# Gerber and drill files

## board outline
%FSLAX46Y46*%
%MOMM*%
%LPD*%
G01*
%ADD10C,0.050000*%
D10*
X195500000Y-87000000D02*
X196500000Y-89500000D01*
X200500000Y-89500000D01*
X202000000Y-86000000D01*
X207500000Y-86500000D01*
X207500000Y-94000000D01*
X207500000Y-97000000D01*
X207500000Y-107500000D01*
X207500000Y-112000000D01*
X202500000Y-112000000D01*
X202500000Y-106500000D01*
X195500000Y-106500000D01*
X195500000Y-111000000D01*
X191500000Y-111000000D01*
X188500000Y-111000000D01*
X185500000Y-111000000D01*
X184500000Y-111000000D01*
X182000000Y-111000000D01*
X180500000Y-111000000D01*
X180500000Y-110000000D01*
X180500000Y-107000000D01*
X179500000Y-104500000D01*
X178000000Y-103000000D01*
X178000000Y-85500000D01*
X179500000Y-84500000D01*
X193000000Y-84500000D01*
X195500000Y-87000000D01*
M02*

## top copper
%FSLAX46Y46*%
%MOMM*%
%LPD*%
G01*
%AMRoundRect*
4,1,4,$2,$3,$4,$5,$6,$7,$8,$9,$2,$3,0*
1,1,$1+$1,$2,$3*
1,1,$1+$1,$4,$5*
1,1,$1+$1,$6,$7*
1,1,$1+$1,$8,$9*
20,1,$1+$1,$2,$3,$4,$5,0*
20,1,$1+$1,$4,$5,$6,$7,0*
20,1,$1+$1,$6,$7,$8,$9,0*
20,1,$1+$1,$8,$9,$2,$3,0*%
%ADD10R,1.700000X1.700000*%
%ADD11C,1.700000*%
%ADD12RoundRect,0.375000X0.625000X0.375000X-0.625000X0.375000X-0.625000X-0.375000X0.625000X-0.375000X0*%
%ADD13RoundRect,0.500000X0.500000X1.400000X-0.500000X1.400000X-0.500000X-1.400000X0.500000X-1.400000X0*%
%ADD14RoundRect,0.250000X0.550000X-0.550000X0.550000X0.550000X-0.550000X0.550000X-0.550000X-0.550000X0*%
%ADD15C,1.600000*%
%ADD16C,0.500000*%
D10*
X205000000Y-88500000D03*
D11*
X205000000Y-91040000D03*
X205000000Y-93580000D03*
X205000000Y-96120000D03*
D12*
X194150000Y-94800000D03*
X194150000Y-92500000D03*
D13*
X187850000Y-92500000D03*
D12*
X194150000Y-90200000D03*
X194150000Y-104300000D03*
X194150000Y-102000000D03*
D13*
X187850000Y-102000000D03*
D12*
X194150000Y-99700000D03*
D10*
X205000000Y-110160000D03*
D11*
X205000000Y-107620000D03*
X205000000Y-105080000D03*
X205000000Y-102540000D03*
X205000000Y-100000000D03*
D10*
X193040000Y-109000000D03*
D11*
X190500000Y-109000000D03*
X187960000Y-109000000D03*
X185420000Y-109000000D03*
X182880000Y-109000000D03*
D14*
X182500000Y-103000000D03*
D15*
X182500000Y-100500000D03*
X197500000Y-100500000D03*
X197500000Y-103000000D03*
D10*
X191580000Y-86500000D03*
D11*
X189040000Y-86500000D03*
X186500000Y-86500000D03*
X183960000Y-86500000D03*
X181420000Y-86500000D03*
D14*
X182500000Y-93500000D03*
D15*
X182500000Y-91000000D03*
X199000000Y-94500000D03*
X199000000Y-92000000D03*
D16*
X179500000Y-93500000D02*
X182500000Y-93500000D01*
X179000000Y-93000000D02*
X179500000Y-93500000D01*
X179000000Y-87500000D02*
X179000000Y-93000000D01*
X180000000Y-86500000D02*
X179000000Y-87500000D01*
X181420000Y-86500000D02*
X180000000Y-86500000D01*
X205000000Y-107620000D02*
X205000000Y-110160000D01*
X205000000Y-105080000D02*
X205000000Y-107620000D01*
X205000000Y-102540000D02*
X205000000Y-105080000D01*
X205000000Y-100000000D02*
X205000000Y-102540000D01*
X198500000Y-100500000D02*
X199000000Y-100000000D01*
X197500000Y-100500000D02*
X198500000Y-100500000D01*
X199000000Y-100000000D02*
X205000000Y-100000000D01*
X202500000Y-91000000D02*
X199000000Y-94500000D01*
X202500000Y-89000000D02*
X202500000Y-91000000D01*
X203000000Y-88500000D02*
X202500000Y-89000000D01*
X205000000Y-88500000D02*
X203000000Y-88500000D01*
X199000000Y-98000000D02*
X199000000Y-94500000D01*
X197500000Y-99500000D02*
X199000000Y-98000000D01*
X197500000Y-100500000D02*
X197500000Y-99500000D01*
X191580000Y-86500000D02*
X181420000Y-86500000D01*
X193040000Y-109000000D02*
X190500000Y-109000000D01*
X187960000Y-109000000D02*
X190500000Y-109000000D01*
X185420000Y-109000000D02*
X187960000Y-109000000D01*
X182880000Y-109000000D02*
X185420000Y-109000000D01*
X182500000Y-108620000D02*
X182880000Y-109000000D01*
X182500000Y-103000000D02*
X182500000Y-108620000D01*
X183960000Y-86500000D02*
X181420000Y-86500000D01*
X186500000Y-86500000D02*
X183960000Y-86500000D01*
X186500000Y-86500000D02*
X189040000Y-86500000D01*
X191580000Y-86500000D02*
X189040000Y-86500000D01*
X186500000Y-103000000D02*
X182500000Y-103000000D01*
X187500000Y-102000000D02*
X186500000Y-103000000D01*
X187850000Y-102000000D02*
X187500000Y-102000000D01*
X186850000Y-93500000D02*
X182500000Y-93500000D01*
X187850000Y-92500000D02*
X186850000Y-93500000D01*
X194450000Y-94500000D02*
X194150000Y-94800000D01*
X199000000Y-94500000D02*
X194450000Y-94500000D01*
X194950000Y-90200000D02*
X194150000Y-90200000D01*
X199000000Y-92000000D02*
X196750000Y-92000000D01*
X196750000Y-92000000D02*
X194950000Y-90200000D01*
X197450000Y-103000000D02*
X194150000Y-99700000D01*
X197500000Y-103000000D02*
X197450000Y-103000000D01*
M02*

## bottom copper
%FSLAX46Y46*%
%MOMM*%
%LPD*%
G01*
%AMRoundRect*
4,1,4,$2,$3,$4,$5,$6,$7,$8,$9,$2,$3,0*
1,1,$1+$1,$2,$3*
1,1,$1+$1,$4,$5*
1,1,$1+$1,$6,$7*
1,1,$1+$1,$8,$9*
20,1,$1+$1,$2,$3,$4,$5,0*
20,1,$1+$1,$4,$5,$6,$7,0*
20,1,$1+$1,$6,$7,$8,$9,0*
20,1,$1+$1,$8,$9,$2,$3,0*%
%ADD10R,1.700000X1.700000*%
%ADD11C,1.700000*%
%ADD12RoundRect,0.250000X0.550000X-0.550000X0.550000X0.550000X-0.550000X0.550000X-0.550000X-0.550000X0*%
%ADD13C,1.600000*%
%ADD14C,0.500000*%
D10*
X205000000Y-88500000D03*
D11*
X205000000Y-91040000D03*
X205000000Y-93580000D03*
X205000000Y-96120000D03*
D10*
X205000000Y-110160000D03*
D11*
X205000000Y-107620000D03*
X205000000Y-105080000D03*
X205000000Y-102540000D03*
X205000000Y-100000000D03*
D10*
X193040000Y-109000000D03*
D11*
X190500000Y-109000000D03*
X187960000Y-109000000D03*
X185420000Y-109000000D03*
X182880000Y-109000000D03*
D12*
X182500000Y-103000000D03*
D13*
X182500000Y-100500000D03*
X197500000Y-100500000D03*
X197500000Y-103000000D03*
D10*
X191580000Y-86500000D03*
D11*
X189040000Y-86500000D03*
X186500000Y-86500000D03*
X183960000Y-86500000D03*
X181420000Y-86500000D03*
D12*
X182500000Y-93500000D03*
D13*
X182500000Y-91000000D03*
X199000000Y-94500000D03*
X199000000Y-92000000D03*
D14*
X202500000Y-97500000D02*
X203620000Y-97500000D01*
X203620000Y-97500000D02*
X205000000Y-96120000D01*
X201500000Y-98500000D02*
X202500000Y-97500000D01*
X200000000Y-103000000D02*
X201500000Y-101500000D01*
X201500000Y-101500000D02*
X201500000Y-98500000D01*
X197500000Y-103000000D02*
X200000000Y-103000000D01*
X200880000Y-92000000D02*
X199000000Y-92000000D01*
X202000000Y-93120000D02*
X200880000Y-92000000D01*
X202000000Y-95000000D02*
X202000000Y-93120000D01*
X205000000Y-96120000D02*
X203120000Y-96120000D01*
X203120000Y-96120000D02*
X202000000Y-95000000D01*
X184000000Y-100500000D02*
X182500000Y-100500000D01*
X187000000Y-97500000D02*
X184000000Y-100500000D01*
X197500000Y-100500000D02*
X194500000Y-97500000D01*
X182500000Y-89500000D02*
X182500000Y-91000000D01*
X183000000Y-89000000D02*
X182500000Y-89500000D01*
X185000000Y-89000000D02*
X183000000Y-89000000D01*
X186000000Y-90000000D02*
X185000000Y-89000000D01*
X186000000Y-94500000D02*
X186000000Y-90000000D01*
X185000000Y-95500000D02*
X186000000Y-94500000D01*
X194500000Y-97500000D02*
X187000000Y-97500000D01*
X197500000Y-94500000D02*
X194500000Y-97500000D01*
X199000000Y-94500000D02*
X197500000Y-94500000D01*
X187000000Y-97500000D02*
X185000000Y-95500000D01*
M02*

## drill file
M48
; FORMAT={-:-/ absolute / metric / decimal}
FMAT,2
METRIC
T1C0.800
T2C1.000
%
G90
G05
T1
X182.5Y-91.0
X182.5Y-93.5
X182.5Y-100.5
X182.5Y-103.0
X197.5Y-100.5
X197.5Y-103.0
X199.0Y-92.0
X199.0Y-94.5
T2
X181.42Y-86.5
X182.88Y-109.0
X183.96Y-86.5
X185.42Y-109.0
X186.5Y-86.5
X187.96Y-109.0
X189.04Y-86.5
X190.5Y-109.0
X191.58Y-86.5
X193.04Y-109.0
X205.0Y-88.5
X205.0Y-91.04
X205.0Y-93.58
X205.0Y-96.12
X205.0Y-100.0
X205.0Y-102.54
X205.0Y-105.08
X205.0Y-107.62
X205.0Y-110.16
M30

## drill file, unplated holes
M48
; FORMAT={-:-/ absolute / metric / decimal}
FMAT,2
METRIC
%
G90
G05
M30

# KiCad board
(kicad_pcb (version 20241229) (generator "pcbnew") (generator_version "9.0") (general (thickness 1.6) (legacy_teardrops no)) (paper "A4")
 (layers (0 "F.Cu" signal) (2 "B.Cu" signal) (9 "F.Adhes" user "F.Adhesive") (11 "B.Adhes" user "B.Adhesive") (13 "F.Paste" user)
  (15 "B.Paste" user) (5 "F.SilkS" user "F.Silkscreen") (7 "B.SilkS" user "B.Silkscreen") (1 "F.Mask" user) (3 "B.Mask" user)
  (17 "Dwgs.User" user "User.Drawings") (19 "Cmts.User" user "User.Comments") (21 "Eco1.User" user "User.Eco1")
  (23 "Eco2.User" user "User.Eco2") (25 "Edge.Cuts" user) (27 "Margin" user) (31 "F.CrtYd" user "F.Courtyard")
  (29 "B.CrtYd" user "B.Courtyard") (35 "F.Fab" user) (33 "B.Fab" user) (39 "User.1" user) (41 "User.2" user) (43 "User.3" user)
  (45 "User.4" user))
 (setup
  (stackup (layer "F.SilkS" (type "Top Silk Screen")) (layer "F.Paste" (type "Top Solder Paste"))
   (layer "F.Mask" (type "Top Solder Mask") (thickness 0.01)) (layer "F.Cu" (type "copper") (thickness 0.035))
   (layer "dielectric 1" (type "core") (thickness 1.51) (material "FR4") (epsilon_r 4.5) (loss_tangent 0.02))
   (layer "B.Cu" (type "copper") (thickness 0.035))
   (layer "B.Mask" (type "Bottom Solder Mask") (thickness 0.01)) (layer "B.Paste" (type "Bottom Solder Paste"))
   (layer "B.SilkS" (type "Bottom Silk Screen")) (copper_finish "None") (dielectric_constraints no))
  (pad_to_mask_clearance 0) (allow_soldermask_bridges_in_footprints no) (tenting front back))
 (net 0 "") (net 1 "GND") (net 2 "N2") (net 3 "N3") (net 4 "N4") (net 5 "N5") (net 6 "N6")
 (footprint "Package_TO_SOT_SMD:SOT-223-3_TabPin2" (layer "F.Cu") (at 191 92.5 180)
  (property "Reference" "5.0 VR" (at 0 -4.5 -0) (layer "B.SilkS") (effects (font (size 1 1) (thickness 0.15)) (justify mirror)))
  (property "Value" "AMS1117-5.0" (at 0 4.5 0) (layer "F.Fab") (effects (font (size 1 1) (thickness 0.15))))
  (pad "1" smd roundrect (at -3.15 -2.3 180) (size 2 1.5) (layers "F.Cu" "F.Mask" "F.Paste") (roundrect_rratio 0.25) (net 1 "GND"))
  (pad "2" smd roundrect (at -3.15 0 180) (size 2 1.5) (layers "F.Cu" "F.Mask" "F.Paste") (roundrect_rratio 0.25) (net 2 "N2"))
  (pad "2" smd roundrect (at 3.15 0 180) (size 2 3.8) (layers "F.Cu" "F.Mask" "F.Paste") (roundrect_rratio 0.25) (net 2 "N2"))
  (pad "3" smd roundrect (at -3.15 2.3 180) (size 2 1.5) (layers "F.Cu" "F.Mask" "F.Paste") (roundrect_rratio 0.25) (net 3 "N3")))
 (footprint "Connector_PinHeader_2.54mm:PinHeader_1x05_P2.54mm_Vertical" (layer "F.Cu") (at 205 110.16 180)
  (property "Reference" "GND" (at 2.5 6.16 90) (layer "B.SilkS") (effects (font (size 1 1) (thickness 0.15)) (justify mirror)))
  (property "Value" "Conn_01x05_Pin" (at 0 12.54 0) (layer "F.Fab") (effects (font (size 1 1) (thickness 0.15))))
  (pad "1" thru_hole rect (at 0 0 180) (size 1.7 1.7) (drill 1) (layers "*.Cu" "*.Mask") (remove_unused_layers no) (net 1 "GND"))
  (pad "2" thru_hole circle (at 0 2.54 180) (size 1.7 1.7) (drill 1) (layers "*.Cu" "*.Mask") (remove_unused_layers no) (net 1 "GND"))
  (pad "3" thru_hole circle (at 0 5.08 180) (size 1.7 1.7) (drill 1) (layers "*.Cu" "*.Mask") (remove_unused_layers no) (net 1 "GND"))
  (pad "4" thru_hole circle (at 0 7.62 180) (size 1.7 1.7) (drill 1) (layers "*.Cu" "*.Mask") (remove_unused_layers no) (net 1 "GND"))
  (pad "5" thru_hole circle (at 0 10.16 180) (size 1.7 1.7) (drill 1) (layers "*.Cu" "*.Mask") (remove_unused_layers no) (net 1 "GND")))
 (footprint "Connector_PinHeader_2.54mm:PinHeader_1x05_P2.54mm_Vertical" (layer "F.Cu") (at 193.04 109 -90)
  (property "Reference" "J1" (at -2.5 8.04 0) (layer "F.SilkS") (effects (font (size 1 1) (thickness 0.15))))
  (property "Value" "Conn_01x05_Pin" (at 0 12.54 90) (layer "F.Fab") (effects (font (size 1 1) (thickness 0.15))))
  (pad "1" thru_hole rect (at 0 0 270) (size 1.7 1.7) (drill 1) (layers "*.Cu" "*.Mask") (remove_unused_layers no) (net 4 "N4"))
  (pad "2" thru_hole circle (at 0 2.54 270) (size 1.7 1.7) (drill 1) (layers "*.Cu" "*.Mask") (remove_unused_layers no) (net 4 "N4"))
  (pad "3" thru_hole circle (at 0 5.08 270) (size 1.7 1.7) (drill 1) (layers "*.Cu" "*.Mask") (remove_unused_layers no) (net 4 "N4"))
  (pad "4" thru_hole circle (at 0 7.62 270) (size 1.7 1.7) (drill 1) (layers "*.Cu" "*.Mask") (remove_unused_layers no) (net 4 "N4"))
  (pad "5" thru_hole circle (at 0 10.16 270) (size 1.7 1.7) (drill 1) (layers "*.Cu" "*.Mask") (remove_unused_layers no) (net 4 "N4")))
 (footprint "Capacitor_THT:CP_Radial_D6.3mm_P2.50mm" (layer "F.Cu") (at 182.5 103 90)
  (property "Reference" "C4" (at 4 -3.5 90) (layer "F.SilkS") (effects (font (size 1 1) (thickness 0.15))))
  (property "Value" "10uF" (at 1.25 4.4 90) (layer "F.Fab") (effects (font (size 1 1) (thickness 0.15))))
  (pad "1" thru_hole roundrect (at 0 0 90) (size 1.6 1.6) (drill 0.8) (layers "*.Cu" "*.Mask") (remove_unused_layers no)
   (roundrect_rratio 0.15625) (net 4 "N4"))
  (pad "2" thru_hole circle (at 2.5 0 90) (size 1.6 1.6) (drill 0.8) (layers "*.Cu" "*.Mask") (remove_unused_layers no) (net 1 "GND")))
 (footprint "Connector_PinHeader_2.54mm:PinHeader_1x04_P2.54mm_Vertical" (layer "F.Cu") (at 205 88.5)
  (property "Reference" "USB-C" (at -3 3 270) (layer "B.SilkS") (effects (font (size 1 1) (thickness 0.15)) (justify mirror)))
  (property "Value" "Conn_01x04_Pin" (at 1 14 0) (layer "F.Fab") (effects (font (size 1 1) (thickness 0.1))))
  (pad "1" thru_hole rect (at 0 0) (size 1.7 1.7) (drill 1) (layers "*.Cu" "*.Mask") (remove_unused_layers no) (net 1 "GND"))
  (pad "2" thru_hole circle (at 0 2.54) (size 1.7 1.7) (drill 1) (layers "*.Cu" "*.Mask") (remove_unused_layers no) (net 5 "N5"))
  (pad "3" thru_hole circle (at 0 5.08) (size 1.7 1.7) (drill 1) (layers "*.Cu" "*.Mask") (remove_unused_layers no) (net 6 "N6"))
  (pad "4" thru_hole circle (at 0 7.62) (size 1.7 1.7) (drill 1) (layers "*.Cu" "*.Mask") (remove_unused_layers no) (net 3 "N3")))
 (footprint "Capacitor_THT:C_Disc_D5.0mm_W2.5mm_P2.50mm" (layer "F.Cu") (at 197.5 100.5 -90)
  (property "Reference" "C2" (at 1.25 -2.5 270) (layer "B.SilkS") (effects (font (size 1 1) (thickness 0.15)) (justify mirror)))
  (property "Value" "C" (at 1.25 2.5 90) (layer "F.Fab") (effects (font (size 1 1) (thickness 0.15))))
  (pad "1" thru_hole circle (at 0 0 270) (size 1.6 1.6) (drill 0.8) (layers "*.Cu" "*.Mask") (remove_unused_layers no) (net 1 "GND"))
  (pad "2" thru_hole circle (at 2.5 0 270) (size 1.6 1.6) (drill 0.8) (layers "*.Cu" "*.Mask") (remove_unused_layers no) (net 3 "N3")))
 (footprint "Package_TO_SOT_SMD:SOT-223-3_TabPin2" (layer "F.Cu") (at 191 102 180)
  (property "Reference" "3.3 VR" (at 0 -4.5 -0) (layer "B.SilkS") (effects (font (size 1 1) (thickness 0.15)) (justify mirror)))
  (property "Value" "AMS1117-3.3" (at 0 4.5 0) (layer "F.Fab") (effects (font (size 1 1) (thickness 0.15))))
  (pad "1" smd roundrect (at -3.15 -2.3 180) (size 2 1.5) (layers "F.Cu" "F.Mask" "F.Paste") (roundrect_rratio 0.25) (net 1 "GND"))
  (pad "2" smd roundrect (at -3.15 0 180) (size 2 1.5) (layers "F.Cu" "F.Mask" "F.Paste") (roundrect_rratio 0.25) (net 4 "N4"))
  (pad "2" smd roundrect (at 3.15 0 180) (size 2 3.8) (layers "F.Cu" "F.Mask" "F.Paste") (roundrect_rratio 0.25) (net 4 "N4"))
  (pad "3" smd roundrect (at -3.15 2.3 180) (size 2 1.5) (layers "F.Cu" "F.Mask" "F.Paste") (roundrect_rratio 0.25) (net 3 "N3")))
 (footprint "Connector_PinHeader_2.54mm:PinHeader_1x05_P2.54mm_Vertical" (layer "F.Cu") (at 191.58 86.5 -90)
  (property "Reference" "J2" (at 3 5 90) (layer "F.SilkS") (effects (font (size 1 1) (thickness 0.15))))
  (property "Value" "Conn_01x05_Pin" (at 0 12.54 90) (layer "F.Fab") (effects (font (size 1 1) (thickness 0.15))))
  (pad "1" thru_hole rect (at 0 0 270) (size 1.7 1.7) (drill 1) (layers "*.Cu" "*.Mask") (remove_unused_layers no) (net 2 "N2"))
  (pad "2" thru_hole circle (at 0 2.54 270) (size 1.7 1.7) (drill 1) (layers "*.Cu" "*.Mask") (remove_unused_layers no) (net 2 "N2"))
  (pad "3" thru_hole circle (at 0 5.08 270) (size 1.7 1.7) (drill 1) (layers "*.Cu" "*.Mask") (remove_unused_layers no) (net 2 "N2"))
  (pad "4" thru_hole circle (at 0 7.62 270) (size 1.7 1.7) (drill 1) (layers "*.Cu" "*.Mask") (remove_unused_layers no) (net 2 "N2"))
  (pad "5" thru_hole circle (at 0 10.16 270) (size 1.7 1.7) (drill 1) (layers "*.Cu" "*.Mask") (remove_unused_layers no) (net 2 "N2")))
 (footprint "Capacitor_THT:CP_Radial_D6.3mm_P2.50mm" (layer "F.Cu") (at 182.5 93.5 90)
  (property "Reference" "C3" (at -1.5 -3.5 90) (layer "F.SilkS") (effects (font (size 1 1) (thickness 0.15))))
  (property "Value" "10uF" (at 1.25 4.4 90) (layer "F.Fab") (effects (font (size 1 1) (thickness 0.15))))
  (pad "1" thru_hole roundrect (at 0 0 90) (size 1.6 1.6) (drill 0.8) (layers "*.Cu" "*.Mask") (remove_unused_layers no)
   (roundrect_rratio 0.15625) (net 2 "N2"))
  (pad "2" thru_hole circle (at 2.5 0 90) (size 1.6 1.6) (drill 0.8) (layers "*.Cu" "*.Mask") (remove_unused_layers no) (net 1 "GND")))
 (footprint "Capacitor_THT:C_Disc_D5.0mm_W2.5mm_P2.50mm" (layer "F.Cu") (at 199 94.5 90)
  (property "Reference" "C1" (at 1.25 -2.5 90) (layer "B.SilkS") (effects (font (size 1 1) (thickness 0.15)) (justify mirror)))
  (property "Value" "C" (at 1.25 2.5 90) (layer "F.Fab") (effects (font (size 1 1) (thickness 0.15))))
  (pad "1" thru_hole circle (at 0 0 90) (size 1.6 1.6) (drill 0.8) (layers "*.Cu" "*.Mask") (remove_unused_layers no) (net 1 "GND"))
  (pad "2" thru_hole circle (at 2.5 0 90) (size 1.6 1.6) (drill 0.8) (layers "*.Cu" "*.Mask") (remove_unused_layers no) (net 3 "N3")))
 (gr_poly
  (pts (xy 207.5 86.5) (xy 207.5 94) (xy 207.5 97) (xy 207.5 107.5) (xy 207.5 107.5) (xy 207.5 112) (xy 202.5 112) (xy 202.5 106.5)
   (xy 195.5 106.5) (xy 195.5 111) (xy 191.5 111) (xy 188.5 111) (xy 185.5 111) (xy 184.5 111) (xy 182 111) (xy 180.5 111) (xy 180.5 110)
   (xy 180.5 107) (xy 179.5 104.5) (xy 178 103) (xy 178 85.5) (xy 179.5 84.5) (xy 193 84.5) (xy 195.5 87) (xy 196.5 89.5) (xy 200.5 89.5)
   (xy 202 86))
  (stroke (width 0.05) (type solid)) (fill no) (layer "Edge.Cuts"))
 (segment (start 199 92) (end 196.75 92) (width 0.5) (layer "F.Cu") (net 3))
 (segment (start 194.95 90.2) (end 194.15 90.2) (width 0.5) (layer "F.Cu") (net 3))
 (segment (start 197.45 103) (end 194.15 99.7) (width 0.5) (layer "F.Cu") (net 3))
 (segment (start 197.5 103) (end 197.45 103) (width 0.5) (layer "F.Cu") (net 3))
 (segment (start 196.75 92) (end 194.95 90.2) (width 0.5) (layer "F.Cu") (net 3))
 (segment (start 200.88 92) (end 199 92) (width 0.5) (layer "B.Cu") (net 3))
 (segment (start 202.5 97.5) (end 203.62 97.5) (width 0.5) (layer "B.Cu") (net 3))
 (segment (start 197.5 103) (end 200 103) (width 0.5) (layer "B.Cu") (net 3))
 (segment (start 200 103) (end 201.5 101.5) (width 0.5) (layer "B.Cu") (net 3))
 (segment (start 202 93.12) (end 200.88 92) (width 0.5) (layer "B.Cu") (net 3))
 (segment (start 202 95) (end 202 93.12) (width 0.5) (layer "B.Cu") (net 3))
 (segment (start 203.62 97.5) (end 205 96.12) (width 0.5) (layer "B.Cu") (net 3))
 (segment (start 205 96.12) (end 203.12 96.12) (width 0.5) (layer "B.Cu") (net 3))
 (segment (start 201.5 98.5) (end 202.5 97.5) (width 0.5) (layer "B.Cu") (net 3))
 (segment (start 201.5 101.5) (end 201.5 98.5) (width 0.5) (layer "B.Cu") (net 3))
 (segment (start 203.12 96.12) (end 202 95) (width 0.5) (layer "B.Cu") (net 3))
 (segment (start 205 105.08) (end 205 107.62) (width 0.5) (layer "F.Cu") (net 1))
 (segment (start 205 102.54) (end 205 105.08) (width 0.5) (layer "F.Cu") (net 1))
 (segment (start 197.5 100.5) (end 198.5 100.5) (width 0.5) (layer "F.Cu") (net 1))
 (segment (start 202.5 89) (end 202.5 91) (width 0.5) (layer "F.Cu") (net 1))
 (segment (start 197.5 99.5) (end 199 98) (width 0.5) (layer "F.Cu") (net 1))
 (segment (start 199 98) (end 199 94.5) (width 0.5) (layer "F.Cu") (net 1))
 (segment (start 197.5 100.5) (end 197.5 99.5) (width 0.5) (layer "F.Cu") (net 1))
 (segment (start 202.5 91) (end 199 94.5) (width 0.5) (layer "F.Cu") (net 1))
 (segment (start 205 100) (end 205 102.54) (width 0.5) (layer "F.Cu") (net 1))
 (segment (start 203 88.5) (end 202.5 89) (width 0.5) (layer "F.Cu") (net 1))
 (segment (start 205 107.62) (end 205 110.16) (width 0.5) (layer "F.Cu") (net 1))
 (segment (start 199 100) (end 205 100) (width 0.5) (layer "F.Cu") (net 1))
 (segment (start 199 94.5) (end 194.45 94.5) (width 0.5) (layer "F.Cu") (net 1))
 (segment (start 205 88.5) (end 203 88.5) (width 0.5) (layer "F.Cu") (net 1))
 (segment (start 194.45 94.5) (end 194.15 94.8) (width 0.5) (layer "F.Cu") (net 1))
 (segment (start 198.5 100.5) (end 199 100) (width 0.5) (layer "F.Cu") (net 1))
 (segment (start 184 100.5) (end 182.5 100.5) (width 0.5) (layer "B.Cu") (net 1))
 (segment (start 183 89) (end 182.5 89.5) (width 0.5) (layer "B.Cu") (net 1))
 (segment (start 187 97.5) (end 184 100.5) (width 0.5) (layer "B.Cu") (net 1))
 (segment (start 185 89) (end 183 89) (width 0.5) (layer "B.Cu") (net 1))
 (segment (start 186 90) (end 185 89) (width 0.5) (layer "B.Cu") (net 1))
 (segment (start 186 94.5) (end 186 90) (width 0.5) (layer "B.Cu") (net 1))
 (segment (start 194.5 97.5) (end 187 97.5) (width 0.5) (layer "B.Cu") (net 1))
 (segment (start 199 94.5) (end 197.5 94.5) (width 0.5) (layer "B.Cu") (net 1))
 (segment (start 187 97.5) (end 185 95.5) (width 0.5) (layer "B.Cu") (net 1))
 (segment (start 197.5 100.5) (end 194.5 97.5) (width 0.5) (layer "B.Cu") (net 1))
 (segment (start 182.5 89.5) (end 182.5 91) (width 0.5) (layer "B.Cu") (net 1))
 (segment (start 185 95.5) (end 186 94.5) (width 0.5) (layer "B.Cu") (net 1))
 (segment (start 197.5 94.5) (end 194.5 97.5) (width 0.5) (layer "B.Cu") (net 1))
 (segment (start 187.5 102) (end 186.5 103) (width 0.5) (layer "F.Cu") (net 4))
 (segment (start 185.42 109) (end 187.96 109) (width 0.5) (layer "F.Cu") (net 4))
 (segment (start 186.5 103) (end 182.5 103) (width 0.5) (layer "F.Cu") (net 4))
 (segment (start 193.04 109) (end 190.5 109) (width 0.5) (layer "F.Cu") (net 4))
 (segment (start 187.85 102) (end 187.5 102) (width 0.5) (layer "F.Cu") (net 4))
 (segment (start 187.96 109) (end 190.5 109) (width 0.5) (layer "F.Cu") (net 4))
 (segment (start 182.88 109) (end 185.42 109) (width 0.5) (layer "F.Cu") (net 4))
 (segment (start 182.5 108.62) (end 182.88 109) (width 0.5) (layer "F.Cu") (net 4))
 (segment (start 182.5 103) (end 182.5 108.62) (width 0.5) (layer "F.Cu") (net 4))
 (segment (start 186.85 93.5) (end 182.5 93.5) (width 0.5) (layer "F.Cu") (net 2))
 (segment (start 191.58 86.5) (end 181.42 86.5) (width 0.5) (layer "F.Cu") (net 2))
 (segment (start 186.5 86.5) (end 183.96 86.5) (width 0.5) (layer "F.Cu") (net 2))
 (segment (start 179 87.5) (end 179 93) (width 0.5) (layer "F.Cu") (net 2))
 (segment (start 191.58 86.5) (end 189.04 86.5) (width 0.5) (layer "F.Cu") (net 2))
 (segment (start 181.42 86.5) (end 180 86.5) (width 0.5) (layer "F.Cu") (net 2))
 (segment (start 186.5 86.5) (end 189.04 86.5) (width 0.5) (layer "F.Cu") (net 2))
 (segment (start 180 86.5) (end 179 87.5) (width 0.5) (layer "F.Cu") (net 2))
 (segment (start 179 93) (end 179.5 93.5) (width 0.5) (layer "F.Cu") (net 2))
 (segment (start 183.96 86.5) (end 181.42 86.5) (width 0.5) (layer "F.Cu") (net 2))
 (segment (start 187.85 92.5) (end 186.85 93.5) (width 0.5) (layer "F.Cu") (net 2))
 (segment (start 179.5 93.5) (end 182.5 93.5) (width 0.5) (layer "F.Cu") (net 2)))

